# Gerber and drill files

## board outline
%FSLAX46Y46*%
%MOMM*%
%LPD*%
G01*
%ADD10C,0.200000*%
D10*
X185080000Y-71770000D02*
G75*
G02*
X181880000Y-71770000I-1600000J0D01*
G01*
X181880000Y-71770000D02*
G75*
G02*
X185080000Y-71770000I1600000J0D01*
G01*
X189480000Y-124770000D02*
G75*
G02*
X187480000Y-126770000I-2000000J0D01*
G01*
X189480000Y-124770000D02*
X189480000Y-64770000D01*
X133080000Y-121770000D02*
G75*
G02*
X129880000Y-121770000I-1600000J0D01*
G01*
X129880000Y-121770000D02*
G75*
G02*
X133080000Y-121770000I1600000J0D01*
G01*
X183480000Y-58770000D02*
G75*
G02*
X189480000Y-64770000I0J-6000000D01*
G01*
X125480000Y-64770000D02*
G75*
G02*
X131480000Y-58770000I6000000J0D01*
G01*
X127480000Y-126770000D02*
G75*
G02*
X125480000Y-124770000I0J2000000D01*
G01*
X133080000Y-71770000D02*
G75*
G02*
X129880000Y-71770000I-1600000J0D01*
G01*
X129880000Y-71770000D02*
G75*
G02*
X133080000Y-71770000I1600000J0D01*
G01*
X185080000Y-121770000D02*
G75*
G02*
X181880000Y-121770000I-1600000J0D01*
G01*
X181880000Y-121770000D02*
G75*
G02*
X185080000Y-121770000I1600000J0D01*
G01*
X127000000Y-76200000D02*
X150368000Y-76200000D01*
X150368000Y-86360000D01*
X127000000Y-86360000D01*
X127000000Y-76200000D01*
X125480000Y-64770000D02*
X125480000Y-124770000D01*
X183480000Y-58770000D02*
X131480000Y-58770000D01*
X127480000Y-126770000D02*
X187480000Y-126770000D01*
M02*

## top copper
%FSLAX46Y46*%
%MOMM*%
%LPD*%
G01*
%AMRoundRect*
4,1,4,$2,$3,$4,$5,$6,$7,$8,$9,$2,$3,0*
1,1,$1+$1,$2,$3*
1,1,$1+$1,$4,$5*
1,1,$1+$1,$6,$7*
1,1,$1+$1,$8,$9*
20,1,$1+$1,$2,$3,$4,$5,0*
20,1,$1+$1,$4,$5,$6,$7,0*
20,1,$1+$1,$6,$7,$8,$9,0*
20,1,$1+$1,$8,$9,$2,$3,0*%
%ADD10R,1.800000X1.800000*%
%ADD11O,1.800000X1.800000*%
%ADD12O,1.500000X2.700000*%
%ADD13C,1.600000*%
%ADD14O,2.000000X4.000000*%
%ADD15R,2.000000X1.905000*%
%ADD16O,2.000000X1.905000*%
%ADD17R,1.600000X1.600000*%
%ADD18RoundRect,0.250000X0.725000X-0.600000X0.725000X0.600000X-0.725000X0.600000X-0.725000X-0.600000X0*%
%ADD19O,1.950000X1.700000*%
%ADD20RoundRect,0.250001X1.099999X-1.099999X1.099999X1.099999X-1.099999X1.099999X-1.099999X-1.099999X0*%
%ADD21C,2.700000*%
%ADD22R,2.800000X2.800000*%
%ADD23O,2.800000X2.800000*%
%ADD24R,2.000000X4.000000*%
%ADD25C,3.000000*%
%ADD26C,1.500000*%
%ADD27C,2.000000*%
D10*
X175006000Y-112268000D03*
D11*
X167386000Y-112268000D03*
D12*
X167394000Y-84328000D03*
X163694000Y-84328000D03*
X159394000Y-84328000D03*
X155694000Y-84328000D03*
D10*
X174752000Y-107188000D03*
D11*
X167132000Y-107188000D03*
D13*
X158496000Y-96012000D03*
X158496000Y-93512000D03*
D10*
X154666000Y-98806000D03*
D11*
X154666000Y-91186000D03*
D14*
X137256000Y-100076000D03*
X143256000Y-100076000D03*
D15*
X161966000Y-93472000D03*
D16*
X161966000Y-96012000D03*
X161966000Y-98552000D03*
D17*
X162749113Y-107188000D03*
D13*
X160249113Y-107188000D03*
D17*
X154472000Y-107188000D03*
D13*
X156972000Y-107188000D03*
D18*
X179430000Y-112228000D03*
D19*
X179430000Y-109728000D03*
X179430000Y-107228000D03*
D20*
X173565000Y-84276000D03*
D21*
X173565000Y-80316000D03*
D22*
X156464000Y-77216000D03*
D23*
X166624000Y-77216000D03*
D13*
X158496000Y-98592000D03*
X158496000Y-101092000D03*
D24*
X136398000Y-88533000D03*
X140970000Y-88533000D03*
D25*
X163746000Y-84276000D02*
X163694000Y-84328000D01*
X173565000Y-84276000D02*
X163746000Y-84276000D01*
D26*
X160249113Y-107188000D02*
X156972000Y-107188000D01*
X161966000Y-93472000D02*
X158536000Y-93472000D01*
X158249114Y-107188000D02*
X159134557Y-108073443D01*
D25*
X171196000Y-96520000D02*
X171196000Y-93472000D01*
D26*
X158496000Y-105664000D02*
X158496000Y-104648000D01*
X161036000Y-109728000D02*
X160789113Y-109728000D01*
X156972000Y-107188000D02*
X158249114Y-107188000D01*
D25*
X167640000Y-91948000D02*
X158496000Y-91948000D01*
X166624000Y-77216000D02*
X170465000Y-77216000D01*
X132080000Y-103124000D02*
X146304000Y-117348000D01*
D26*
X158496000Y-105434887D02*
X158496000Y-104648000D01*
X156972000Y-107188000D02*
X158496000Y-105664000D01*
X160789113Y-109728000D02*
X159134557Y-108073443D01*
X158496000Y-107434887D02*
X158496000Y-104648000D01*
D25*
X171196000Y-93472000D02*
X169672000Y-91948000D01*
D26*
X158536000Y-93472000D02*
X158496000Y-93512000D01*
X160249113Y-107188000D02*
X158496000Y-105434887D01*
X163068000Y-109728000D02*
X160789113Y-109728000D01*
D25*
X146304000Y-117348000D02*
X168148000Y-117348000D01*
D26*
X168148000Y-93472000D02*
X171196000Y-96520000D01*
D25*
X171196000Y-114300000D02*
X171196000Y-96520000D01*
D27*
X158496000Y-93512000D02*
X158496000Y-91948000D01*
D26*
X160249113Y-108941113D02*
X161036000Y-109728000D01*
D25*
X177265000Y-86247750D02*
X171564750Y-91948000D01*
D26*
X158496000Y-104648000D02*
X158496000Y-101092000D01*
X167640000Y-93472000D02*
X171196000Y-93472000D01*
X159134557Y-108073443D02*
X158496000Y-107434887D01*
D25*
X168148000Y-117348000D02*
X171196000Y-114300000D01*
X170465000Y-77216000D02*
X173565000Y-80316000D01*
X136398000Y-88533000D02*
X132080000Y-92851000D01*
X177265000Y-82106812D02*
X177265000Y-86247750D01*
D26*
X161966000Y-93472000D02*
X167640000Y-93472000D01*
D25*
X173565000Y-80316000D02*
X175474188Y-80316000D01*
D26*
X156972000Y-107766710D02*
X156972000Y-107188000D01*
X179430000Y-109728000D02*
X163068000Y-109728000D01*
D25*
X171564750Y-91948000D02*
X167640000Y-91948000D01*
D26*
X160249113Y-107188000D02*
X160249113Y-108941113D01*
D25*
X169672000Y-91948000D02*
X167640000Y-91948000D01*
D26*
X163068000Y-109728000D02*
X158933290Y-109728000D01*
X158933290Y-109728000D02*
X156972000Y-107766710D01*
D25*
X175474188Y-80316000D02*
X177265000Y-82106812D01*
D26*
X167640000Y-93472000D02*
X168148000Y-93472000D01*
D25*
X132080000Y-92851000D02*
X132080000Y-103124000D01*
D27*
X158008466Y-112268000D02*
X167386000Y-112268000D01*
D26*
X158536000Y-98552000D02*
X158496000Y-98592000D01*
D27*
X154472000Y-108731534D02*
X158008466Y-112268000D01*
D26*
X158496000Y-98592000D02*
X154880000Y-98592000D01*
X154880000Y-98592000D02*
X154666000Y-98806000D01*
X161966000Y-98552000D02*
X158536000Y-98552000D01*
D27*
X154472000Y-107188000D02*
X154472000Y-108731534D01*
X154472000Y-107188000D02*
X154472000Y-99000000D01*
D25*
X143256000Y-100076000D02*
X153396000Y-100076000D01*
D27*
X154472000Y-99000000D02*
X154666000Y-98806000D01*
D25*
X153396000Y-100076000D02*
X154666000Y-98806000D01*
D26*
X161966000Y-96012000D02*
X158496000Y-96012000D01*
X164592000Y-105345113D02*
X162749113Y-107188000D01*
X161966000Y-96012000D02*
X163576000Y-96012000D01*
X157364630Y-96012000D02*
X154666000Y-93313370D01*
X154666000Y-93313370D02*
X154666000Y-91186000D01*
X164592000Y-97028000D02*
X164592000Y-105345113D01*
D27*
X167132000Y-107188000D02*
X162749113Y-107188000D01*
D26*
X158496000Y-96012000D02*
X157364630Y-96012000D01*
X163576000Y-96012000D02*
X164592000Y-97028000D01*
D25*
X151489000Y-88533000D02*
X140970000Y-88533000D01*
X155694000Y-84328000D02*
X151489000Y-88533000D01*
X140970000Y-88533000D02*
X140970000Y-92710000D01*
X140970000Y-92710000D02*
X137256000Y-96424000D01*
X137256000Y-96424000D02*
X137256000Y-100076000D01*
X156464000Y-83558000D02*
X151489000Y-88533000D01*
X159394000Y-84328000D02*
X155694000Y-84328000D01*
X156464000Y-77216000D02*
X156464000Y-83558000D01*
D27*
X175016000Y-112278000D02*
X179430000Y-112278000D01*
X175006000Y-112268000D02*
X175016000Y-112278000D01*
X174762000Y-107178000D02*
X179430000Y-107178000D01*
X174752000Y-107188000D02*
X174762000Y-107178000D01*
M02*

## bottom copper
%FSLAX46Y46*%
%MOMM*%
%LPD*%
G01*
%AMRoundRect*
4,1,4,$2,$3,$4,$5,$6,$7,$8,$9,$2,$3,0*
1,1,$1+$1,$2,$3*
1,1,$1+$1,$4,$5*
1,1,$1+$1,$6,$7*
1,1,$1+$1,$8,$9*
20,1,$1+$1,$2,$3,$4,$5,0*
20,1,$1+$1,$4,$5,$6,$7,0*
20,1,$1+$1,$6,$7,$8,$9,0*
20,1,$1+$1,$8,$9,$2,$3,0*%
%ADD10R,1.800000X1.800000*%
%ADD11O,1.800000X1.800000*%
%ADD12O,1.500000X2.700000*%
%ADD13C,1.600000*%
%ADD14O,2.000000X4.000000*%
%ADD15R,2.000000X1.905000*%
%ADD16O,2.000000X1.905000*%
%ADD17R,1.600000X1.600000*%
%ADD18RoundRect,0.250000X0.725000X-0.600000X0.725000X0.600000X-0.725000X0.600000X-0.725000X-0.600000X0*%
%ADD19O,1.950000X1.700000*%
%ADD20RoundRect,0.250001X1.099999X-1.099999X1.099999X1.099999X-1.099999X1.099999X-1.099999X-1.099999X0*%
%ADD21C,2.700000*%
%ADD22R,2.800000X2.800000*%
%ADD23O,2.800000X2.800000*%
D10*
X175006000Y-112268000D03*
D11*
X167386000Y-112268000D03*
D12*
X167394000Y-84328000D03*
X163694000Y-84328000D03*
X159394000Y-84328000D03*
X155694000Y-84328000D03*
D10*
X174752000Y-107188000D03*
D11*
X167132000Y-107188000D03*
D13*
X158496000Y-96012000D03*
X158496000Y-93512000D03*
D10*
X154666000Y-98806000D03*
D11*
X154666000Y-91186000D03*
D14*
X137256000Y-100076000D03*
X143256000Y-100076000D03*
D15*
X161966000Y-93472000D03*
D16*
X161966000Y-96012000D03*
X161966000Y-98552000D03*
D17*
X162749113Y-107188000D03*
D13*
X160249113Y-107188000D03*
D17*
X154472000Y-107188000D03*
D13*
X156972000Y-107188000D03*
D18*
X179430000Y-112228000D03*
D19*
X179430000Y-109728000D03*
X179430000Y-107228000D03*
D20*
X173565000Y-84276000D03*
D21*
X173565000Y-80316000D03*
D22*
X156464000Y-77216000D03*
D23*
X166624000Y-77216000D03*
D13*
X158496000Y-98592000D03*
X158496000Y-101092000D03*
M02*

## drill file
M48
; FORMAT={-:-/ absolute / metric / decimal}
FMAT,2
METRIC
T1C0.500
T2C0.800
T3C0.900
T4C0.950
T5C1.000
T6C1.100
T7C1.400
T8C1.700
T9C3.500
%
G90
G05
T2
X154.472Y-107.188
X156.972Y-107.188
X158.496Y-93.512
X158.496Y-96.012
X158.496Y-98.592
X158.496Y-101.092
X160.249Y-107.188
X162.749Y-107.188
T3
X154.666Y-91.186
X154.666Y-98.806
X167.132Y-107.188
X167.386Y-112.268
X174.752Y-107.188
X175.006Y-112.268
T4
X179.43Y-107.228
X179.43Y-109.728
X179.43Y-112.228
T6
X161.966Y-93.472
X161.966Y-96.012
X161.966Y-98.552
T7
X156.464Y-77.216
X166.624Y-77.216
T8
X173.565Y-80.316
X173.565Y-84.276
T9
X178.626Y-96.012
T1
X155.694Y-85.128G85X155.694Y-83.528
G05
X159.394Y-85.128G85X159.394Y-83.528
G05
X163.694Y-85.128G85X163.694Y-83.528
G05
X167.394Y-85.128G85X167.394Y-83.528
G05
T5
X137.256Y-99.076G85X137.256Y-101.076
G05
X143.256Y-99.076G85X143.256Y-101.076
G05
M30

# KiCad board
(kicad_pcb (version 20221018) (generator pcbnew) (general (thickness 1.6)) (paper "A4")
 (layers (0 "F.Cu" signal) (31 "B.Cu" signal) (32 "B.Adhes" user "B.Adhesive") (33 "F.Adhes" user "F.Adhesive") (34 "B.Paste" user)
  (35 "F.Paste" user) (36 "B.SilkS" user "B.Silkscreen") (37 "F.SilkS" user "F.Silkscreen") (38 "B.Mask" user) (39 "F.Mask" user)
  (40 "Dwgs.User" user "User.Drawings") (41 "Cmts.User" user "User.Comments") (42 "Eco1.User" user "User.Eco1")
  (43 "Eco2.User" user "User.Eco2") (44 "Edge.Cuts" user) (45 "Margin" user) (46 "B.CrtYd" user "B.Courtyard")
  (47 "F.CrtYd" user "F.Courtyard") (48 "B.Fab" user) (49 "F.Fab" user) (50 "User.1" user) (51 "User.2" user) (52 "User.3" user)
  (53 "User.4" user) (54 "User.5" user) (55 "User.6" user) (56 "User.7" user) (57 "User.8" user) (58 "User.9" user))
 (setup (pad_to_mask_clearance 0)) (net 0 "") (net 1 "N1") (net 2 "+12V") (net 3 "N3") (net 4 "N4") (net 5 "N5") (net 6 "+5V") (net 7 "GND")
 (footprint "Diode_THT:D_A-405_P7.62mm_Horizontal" (layer "F.Cu") (at 175.006 112.268 180)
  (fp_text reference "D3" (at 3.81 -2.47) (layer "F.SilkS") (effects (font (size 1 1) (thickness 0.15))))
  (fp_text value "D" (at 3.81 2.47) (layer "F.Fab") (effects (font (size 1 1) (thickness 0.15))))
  (pad "1" thru_hole rect (at 0 0 180) (size 1.8 1.8) (drill 0.9) (layers "*.Cu" "*.Mask") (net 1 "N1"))
  (pad "2" thru_hole oval (at 7.62 0 180) (size 1.8 1.8) (drill 0.9) (layers "*.Cu" "*.Mask") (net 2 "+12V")))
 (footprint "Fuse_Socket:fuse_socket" (layer "F.Cu") (at 161.544 86.868 180)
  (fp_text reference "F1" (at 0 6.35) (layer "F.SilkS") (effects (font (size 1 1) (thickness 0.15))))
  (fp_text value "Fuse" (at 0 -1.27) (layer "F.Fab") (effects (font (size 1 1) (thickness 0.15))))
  (pad "1" thru_hole oval (at -5.85 2.54 180) (size 1.5 2.7) (drill oval 0.5 2.1) (layers "*.Cu" "*.Mask") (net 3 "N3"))
  (pad "1" thru_hole oval (at -2.15 2.54 180) (size 1.5 2.7) (drill oval 0.5 2.1) (layers "*.Cu" "*.Mask") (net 3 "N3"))
  (pad "2" thru_hole oval (at 2.15 2.54 180) (size 1.5 2.7) (drill oval 0.5 2.1) (layers "*.Cu" "*.Mask") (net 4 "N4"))
  (pad "2" thru_hole oval (at 5.85 2.54 180) (size 1.5 2.7) (drill oval 0.5 2.1) (layers "*.Cu" "*.Mask") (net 4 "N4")))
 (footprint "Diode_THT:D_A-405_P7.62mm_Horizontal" (layer "F.Cu") (at 174.752 107.188 180)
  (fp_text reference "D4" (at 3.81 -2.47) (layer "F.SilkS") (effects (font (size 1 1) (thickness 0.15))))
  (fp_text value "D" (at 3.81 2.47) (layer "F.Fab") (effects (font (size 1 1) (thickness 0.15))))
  (pad "1" thru_hole rect (at 0 0 180) (size 1.8 1.8) (drill 0.9) (layers "*.Cu" "*.Mask") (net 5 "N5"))
  (pad "2" thru_hole oval (at 7.62 0 180) (size 1.8 1.8) (drill 0.9) (layers "*.Cu" "*.Mask") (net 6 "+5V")))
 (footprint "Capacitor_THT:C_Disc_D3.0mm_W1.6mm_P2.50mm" (layer "F.Cu") (at 158.496 96.012 90)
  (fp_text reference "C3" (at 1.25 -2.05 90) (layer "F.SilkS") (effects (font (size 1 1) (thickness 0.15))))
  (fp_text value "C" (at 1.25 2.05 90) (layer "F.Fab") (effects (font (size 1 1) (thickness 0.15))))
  (pad "1" thru_hole circle (at 0 0 90) (size 1.6 1.6) (drill 0.8) (layers "*.Cu" "*.Mask") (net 6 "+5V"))
  (pad "2" thru_hole circle (at 2.5 0 90) (size 1.6 1.6) (drill 0.8) (layers "*.Cu" "*.Mask") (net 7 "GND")))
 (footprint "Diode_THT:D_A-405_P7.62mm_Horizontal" (layer "F.Cu") (at 154.666 98.806 90)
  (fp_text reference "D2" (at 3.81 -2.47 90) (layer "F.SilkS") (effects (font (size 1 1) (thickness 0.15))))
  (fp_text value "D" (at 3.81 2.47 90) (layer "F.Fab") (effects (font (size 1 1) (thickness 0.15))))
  (pad "1" thru_hole rect (at 0 0 90) (size 1.8 1.8) (drill 0.9) (layers "*.Cu" "*.Mask") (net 2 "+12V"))
  (pad "2" thru_hole oval (at 7.62 0 90) (size 1.8 1.8) (drill 0.9) (layers "*.Cu" "*.Mask") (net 6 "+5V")))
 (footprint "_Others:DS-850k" (layer "F.Cu") (at 137.256 100.076 180)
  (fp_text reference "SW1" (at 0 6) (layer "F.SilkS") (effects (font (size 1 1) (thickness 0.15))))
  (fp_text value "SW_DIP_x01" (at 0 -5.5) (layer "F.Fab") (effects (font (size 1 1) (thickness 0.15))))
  (pad "1" thru_hole oval (at 0 0 270) (size 4 2) (drill oval 3 1) (layers "*.Cu" "*.Mask") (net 4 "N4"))
  (pad "2" thru_hole oval (at -6 0 270) (size 4 2) (drill oval 3 1) (layers "*.Cu" "*.Mask") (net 2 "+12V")))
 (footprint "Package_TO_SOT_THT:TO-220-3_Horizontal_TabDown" (layer "F.Cu") (at 161.966 93.472 -90)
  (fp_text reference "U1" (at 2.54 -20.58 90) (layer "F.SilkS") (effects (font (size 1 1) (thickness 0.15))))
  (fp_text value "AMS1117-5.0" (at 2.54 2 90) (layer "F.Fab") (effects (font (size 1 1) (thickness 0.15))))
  (pad "" np_thru_hole oval (at 2.54 -16.66 270) (size 3.5 3.5) (drill 3.5) (layers "*.Cu" "*.Mask"))
  (pad "1" thru_hole rect (at 0 0 270) (size 1.905 2) (drill 1.1) (layers "*.Cu" "*.Mask") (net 7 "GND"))
  (pad "2" thru_hole oval (at 2.54 0 270) (size 1.905 2) (drill 1.1) (layers "*.Cu" "*.Mask") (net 6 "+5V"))
  (pad "3" thru_hole oval (at 5.08 0 270) (size 1.905 2) (drill 1.1) (layers "*.Cu" "*.Mask") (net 2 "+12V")))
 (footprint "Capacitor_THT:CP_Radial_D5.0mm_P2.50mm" (layer "F.Cu") (at 162.749113 107.188 180)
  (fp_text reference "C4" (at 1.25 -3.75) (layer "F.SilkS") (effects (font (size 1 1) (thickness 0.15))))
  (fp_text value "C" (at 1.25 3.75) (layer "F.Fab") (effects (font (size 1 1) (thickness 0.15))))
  (pad "1" thru_hole rect (at 0 0 180) (size 1.6 1.6) (drill 0.8) (layers "*.Cu" "*.Mask") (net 6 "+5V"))
  (pad "2" thru_hole circle (at 2.5 0 180) (size 1.6 1.6) (drill 0.8) (layers "*.Cu" "*.Mask") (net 7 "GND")))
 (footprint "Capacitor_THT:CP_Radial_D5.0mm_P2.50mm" (layer "F.Cu") (at 154.472 107.188)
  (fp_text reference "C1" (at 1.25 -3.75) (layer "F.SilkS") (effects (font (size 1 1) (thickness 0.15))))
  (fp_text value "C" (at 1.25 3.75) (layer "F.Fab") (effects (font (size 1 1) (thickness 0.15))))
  (pad "1" thru_hole rect (at 0 0) (size 1.6 1.6) (drill 0.8) (layers "*.Cu" "*.Mask") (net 2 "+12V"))
  (pad "2" thru_hole circle (at 2.5 0) (size 1.6 1.6) (drill 0.8) (layers "*.Cu" "*.Mask") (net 7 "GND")))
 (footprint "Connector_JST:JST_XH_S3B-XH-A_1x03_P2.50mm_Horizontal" (layer "F.Cu") (at 179.43 112.228 90)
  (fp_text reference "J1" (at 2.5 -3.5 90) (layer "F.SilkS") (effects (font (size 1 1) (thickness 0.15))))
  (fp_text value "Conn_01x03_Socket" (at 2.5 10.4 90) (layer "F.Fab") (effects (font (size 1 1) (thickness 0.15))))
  (pad "1" thru_hole roundrect (at 0 0 90) (size 1.7 1.95) (drill 0.95) (layers "*.Cu" "*.Mask") (roundrect_rratio 0.147059) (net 1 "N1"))
  (pad "2" thru_hole oval (at 2.5 0 90) (size 1.7 1.95) (drill 0.95) (layers "*.Cu" "*.Mask") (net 7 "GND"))
  (pad "3" thru_hole oval (at 5 0 90) (size 1.7 1.95) (drill 0.95) (layers "*.Cu" "*.Mask") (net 5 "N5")))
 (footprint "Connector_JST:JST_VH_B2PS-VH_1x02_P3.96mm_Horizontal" (layer "F.Cu") (at 173.565 84.276 90)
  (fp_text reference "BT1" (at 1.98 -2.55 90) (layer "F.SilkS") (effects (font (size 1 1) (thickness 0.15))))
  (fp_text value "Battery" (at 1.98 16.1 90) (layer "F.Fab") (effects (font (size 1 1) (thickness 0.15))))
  (pad "1" thru_hole roundrect (at 0 0 90) (size 2.7 2.7) (drill 1.7) (layers "*.Cu" "*.Mask") (roundrect_rratio 0.092593) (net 3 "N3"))
  (pad "2" thru_hole circle (at 3.96 0 90) (size 2.7 2.7) (drill 1.7) (layers "*.Cu" "*.Mask") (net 7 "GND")))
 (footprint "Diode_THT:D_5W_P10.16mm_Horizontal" (layer "F.Cu") (at 156.464 77.216)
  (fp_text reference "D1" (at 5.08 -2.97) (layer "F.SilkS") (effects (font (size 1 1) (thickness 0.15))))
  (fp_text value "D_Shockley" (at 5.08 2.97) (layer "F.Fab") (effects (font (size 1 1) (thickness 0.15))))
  (pad "1" thru_hole rect (at 0 0) (size 2.8 2.8) (drill 1.4) (layers "*.Cu" "*.Mask") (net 4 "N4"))
  (pad "2" thru_hole oval (at 10.16 0) (size 2.8 2.8) (drill 1.4) (layers "*.Cu" "*.Mask") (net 7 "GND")))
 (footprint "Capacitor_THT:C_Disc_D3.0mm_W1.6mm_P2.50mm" (layer "F.Cu") (at 158.496 98.592 -90)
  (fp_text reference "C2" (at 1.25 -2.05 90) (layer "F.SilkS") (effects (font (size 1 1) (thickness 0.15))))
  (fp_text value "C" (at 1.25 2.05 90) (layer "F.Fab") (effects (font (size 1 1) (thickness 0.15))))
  (pad "1" thru_hole circle (at 0 0 270) (size 1.6 1.6) (drill 0.8) (layers "*.Cu" "*.Mask") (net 2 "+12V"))
  (pad "2" thru_hole circle (at 2.5 0 270) (size 1.6 1.6) (drill 0.8) (layers "*.Cu" "*.Mask") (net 7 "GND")))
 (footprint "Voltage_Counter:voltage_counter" (layer "B.Cu") (at 138.684 76.341 180)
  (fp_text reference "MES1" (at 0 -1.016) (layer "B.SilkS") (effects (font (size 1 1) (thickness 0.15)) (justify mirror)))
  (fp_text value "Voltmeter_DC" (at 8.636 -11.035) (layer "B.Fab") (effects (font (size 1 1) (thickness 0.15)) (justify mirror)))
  (pad "1" smd rect (at 2.286 -12.192 180) (size 2 4) (layers "F.Cu" "F.Paste" "F.Mask") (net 7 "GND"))
  (pad "2" smd rect (at -2.286 -12.192 180) (size 2 4) (layers "F.Cu" "F.Paste" "F.Mask") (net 4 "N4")))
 (gr_circle (center 183.48 71.77) (end 181.88 71.77) (stroke (width 0.2) (type solid)) (fill none) (layer "Edge.Cuts"))
 (gr_arc (start 189.48 124.77) (mid 188.894214 126.184214) (end 187.48 126.77) (stroke (width 0.2) (type solid)) (layer "Edge.Cuts"))
 (gr_line (start 189.48 124.77) (end 189.48 64.77) (stroke (width 0.2) (type solid)) (layer "Edge.Cuts"))
 (gr_circle (center 131.48 121.77) (end 129.88 121.77) (stroke (width 0.2) (type solid)) (fill none) (layer "Edge.Cuts"))
 (gr_arc (start 183.48 58.77) (mid 187.722641 60.527359) (end 189.48 64.77) (stroke (width 0.2) (type solid)) (layer "Edge.Cuts"))
 (gr_arc (start 125.48 64.77) (mid 127.237359 60.527359) (end 131.48 58.77) (stroke (width 0.2) (type solid)) (layer "Edge.Cuts"))
 (gr_arc (start 127.48 126.77) (mid 126.065786 126.184214) (end 125.48 124.77) (stroke (width 0.2) (type solid)) (layer "Edge.Cuts"))
 (gr_circle (center 131.48 71.77) (end 129.88 71.77) (stroke (width 0.2) (type solid)) (fill none) (layer "Edge.Cuts"))
 (gr_circle (center 183.48 121.77) (end 181.88 121.77) (stroke (width 0.2) (type solid)) (fill none) (layer "Edge.Cuts"))
 (gr_rect (start 127 76.2) (end 150.368 86.36) (stroke (width 0.2) (type default)) (fill none) (layer "Edge.Cuts"))
 (gr_line (start 125.48 64.77) (end 125.48 124.77) (stroke (width 0.2) (type solid)) (layer "Edge.Cuts"))
 (gr_line (start 183.48 58.77) (end 131.48 58.77) (stroke (width 0.2) (type solid)) (layer "Edge.Cuts"))
 (gr_line (start 127.48 126.77) (end 187.48 126.77) (stroke (width 0.2) (type solid)) (layer "Edge.Cuts"))
 (segment (start 163.746 84.276) (end 163.694 84.328) (width 3) (layer "F.Cu") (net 3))
 (segment (start 173.565 84.276) (end 163.746 84.276) (width 3) (layer "F.Cu") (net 3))
 (segment (start 160.249113 107.188) (end 156.972 107.188) (width 1.5) (layer "F.Cu") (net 7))
 (segment (start 161.966 93.472) (end 158.536 93.472) (width 1.5) (layer "F.Cu") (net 7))
 (segment (start 158.249114 107.188) (end 159.134557 108.073443) (width 1.5) (layer "F.Cu") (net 7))
 (segment (start 171.196 96.52) (end 171.196 93.472) (width 3) (layer "F.Cu") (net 7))
 (segment (start 158.496 105.664) (end 158.496 104.648) (width 1.5) (layer "F.Cu") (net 7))
 (segment (start 161.036 109.728) (end 160.789113 109.728) (width 1.5) (layer "F.Cu") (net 7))
 (segment (start 156.972 107.188) (end 158.249114 107.188) (width 1.5) (layer "F.Cu") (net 7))
 (segment (start 167.64 91.948) (end 158.496 91.948) (width 3) (layer "F.Cu") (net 7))
 (segment (start 166.624 77.216) (end 170.465 77.216) (width 3) (layer "F.Cu") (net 7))
 (segment (start 132.08 103.124) (end 146.304 117.348) (width 3) (layer "F.Cu") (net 7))
 (segment (start 158.496 105.434887) (end 158.496 104.648) (width 1.5) (layer "F.Cu") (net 7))
 (segment (start 156.972 107.188) (end 158.496 105.664) (width 1.5) (layer "F.Cu") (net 7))
 (segment (start 160.789113 109.728) (end 159.134557 108.073443) (width 1.5) (layer "F.Cu") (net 7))
 (segment (start 158.496 107.434887) (end 158.496 104.648) (width 1.5) (layer "F.Cu") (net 7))
 (segment (start 171.196 93.472) (end 169.672 91.948) (width 3) (layer "F.Cu") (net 7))
 (segment (start 158.536 93.472) (end 158.496 93.512) (width 1.5) (layer "F.Cu") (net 7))
 (segment (start 160.249113 107.188) (end 158.496 105.434887) (width 1.5) (layer "F.Cu") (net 7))
 (segment (start 163.068 109.728) (end 160.789113 109.728) (width 1.5) (layer "F.Cu") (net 7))
 (segment (start 146.304 117.348) (end 168.148 117.348) (width 3) (layer "F.Cu") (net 7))
 (segment (start 168.148 93.472) (end 171.196 96.52) (width 1.5) (layer "F.Cu") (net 7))
 (segment (start 171.196 114.3) (end 171.196 96.52) (width 3) (layer "F.Cu") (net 7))
 (segment (start 158.496 93.512) (end 158.496 91.948) (width 2) (layer "F.Cu") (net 7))
 (segment (start 160.249113 108.941113) (end 161.036 109.728) (width 1.5) (layer "F.Cu") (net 7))
 (segment (start 177.265 86.24775) (end 171.56475 91.948) (width 3) (layer "F.Cu") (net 7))
 (segment (start 158.496 104.648) (end 158.496 101.092) (width 1.5) (layer "F.Cu") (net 7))
 (segment (start 167.64 93.472) (end 171.196 93.472) (width 1.5) (layer "F.Cu") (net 7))
 (segment (start 159.134557 108.073443) (end 158.496 107.434887) (width 1.5) (layer "F.Cu") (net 7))
 (segment (start 168.148 117.348) (end 171.196 114.3) (width 3) (layer "F.Cu") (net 7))
 (segment (start 170.465 77.216) (end 173.565 80.316) (width 3) (layer "F.Cu") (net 7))
 (segment (start 136.398 88.533) (end 132.08 92.851) (width 3) (layer "F.Cu") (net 7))
 (segment (start 177.265 82.106812) (end 177.265 86.24775) (width 3) (layer "F.Cu") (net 7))
 (segment (start 161.966 93.472) (end 167.64 93.472) (width 1.5) (layer "F.Cu") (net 7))
 (segment (start 173.565 80.316) (end 175.474188 80.316) (width 3) (layer "F.Cu") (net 7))
 (segment (start 156.972 107.76671) (end 156.972 107.188) (width 1.5) (layer "F.Cu") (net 7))
 (segment (start 179.43 109.728) (end 163.068 109.728) (width 1.5) (layer "F.Cu") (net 7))
 (segment (start 171.56475 91.948) (end 167.64 91.948) (width 3) (layer "F.Cu") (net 7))
 (segment (start 160.249113 107.188) (end 160.249113 108.941113) (width 1.5) (layer "F.Cu") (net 7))
 (segment (start 169.672 91.948) (end 167.64 91.948) (width 3) (layer "F.Cu") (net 7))
 (segment (start 163.068 109.728) (end 158.93329 109.728) (width 1.5) (layer "F.Cu") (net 7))
 (segment (start 158.93329 109.728) (end 156.972 107.76671) (width 1.5) (layer "F.Cu") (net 7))
 (segment (start 175.474188 80.316) (end 177.265 82.106812) (width 3) (layer "F.Cu") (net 7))
 (segment (start 167.64 93.472) (end 168.148 93.472) (width 1.5) (layer "F.Cu") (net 7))
 (segment (start 132.08 92.851) (end 132.08 103.124) (width 3) (layer "F.Cu") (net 7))
 (segment (start 158.008466 112.268) (end 167.386 112.268) (width 2) (layer "F.Cu") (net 2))
 (segment (start 158.536 98.552) (end 158.496 98.592) (width 1.5) (layer "F.Cu") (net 2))
 (segment (start 154.472 108.731534) (end 158.008466 112.268) (width 2) (layer "F.Cu") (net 2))
 (segment (start 158.496 98.592) (end 154.88 98.592) (width 1.5) (layer "F.Cu") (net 2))
 (segment (start 154.88 98.592) (end 154.666 98.806) (width 1.5) (layer "F.Cu") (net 2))
 (segment (start 161.966 98.552) (end 158.536 98.552) (width 1.5) (layer "F.Cu") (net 2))
 (segment (start 154.472 107.188) (end 154.472 108.731534) (width 2) (layer "F.Cu") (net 2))
 (segment (start 154.472 107.188) (end 154.472 99) (width 2) (layer "F.Cu") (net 2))
 (segment (start 143.256 100.076) (end 153.396 100.076) (width 3) (layer "F.Cu") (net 2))
 (segment (start 154.472 99) (end 154.666 98.806) (width 2) (layer "F.Cu") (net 2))
 (segment (start 153.396 100.076) (end 154.666 98.806) (width 3) (layer "F.Cu") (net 2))
 (segment (start 161.966 96.012) (end 158.496 96.012) (width 1.5) (layer "F.Cu") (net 6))
 (segment (start 164.592 105.345113) (end 162.749113 107.188) (width 1.5) (layer "F.Cu") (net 6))
 (segment (start 161.966 96.012) (end 163.576 96.012) (width 1.5) (layer "F.Cu") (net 6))
 (segment (start 157.36463 96.012) (end 154.666 93.31337) (width 1.5) (layer "F.Cu") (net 6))
 (segment (start 154.666 93.31337) (end 154.666 91.186) (width 1.5) (layer "F.Cu") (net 6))
 (segment (start 164.592 97.028) (end 164.592 105.345113) (width 1.5) (layer "F.Cu") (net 6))
 (segment (start 167.132 107.188) (end 162.749113 107.188) (width 2) (layer "F.Cu") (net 6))
 (segment (start 158.496 96.012) (end 157.36463 96.012) (width 1.5) (layer "F.Cu") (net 6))
 (segment (start 163.576 96.012) (end 164.592 97.028) (width 1.5) (layer "F.Cu") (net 6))
 (segment (start 151.489 88.533) (end 140.97 88.533) (width 3) (layer "F.Cu") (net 4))
 (segment (start 155.694 84.328) (end 151.489 88.533) (width 3) (layer "F.Cu") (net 4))
 (segment (start 140.97 88.533) (end 140.97 92.71) (width 3) (layer "F.Cu") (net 4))
 (segment (start 140.97 92.71) (end 137.256 96.424) (width 3) (layer "F.Cu") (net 4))
 (segment (start 137.256 96.424) (end 137.256 100.076) (width 3) (layer "F.Cu") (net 4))
 (segment (start 156.464 83.558) (end 151.489 88.533) (width 3) (layer "F.Cu") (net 4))
 (segment (start 159.394 84.328) (end 155.694 84.328) (width 3) (layer "F.Cu") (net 4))
 (segment (start 156.464 77.216) (end 156.464 83.558) (width 3) (layer "F.Cu") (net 4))
 (segment (start 175.016 112.278) (end 179.43 112.278) (width 2) (layer "F.Cu") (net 1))
 (segment (start 175.006 112.268) (end 175.016 112.278) (width 2) (layer "F.Cu") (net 1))
 (segment (start 174.762 107.178) (end 179.43 107.178) (width 2) (layer "F.Cu") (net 5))
 (segment (start 174.752 107.188) (end 174.762 107.178) (width 2) (layer "F.Cu") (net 5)))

